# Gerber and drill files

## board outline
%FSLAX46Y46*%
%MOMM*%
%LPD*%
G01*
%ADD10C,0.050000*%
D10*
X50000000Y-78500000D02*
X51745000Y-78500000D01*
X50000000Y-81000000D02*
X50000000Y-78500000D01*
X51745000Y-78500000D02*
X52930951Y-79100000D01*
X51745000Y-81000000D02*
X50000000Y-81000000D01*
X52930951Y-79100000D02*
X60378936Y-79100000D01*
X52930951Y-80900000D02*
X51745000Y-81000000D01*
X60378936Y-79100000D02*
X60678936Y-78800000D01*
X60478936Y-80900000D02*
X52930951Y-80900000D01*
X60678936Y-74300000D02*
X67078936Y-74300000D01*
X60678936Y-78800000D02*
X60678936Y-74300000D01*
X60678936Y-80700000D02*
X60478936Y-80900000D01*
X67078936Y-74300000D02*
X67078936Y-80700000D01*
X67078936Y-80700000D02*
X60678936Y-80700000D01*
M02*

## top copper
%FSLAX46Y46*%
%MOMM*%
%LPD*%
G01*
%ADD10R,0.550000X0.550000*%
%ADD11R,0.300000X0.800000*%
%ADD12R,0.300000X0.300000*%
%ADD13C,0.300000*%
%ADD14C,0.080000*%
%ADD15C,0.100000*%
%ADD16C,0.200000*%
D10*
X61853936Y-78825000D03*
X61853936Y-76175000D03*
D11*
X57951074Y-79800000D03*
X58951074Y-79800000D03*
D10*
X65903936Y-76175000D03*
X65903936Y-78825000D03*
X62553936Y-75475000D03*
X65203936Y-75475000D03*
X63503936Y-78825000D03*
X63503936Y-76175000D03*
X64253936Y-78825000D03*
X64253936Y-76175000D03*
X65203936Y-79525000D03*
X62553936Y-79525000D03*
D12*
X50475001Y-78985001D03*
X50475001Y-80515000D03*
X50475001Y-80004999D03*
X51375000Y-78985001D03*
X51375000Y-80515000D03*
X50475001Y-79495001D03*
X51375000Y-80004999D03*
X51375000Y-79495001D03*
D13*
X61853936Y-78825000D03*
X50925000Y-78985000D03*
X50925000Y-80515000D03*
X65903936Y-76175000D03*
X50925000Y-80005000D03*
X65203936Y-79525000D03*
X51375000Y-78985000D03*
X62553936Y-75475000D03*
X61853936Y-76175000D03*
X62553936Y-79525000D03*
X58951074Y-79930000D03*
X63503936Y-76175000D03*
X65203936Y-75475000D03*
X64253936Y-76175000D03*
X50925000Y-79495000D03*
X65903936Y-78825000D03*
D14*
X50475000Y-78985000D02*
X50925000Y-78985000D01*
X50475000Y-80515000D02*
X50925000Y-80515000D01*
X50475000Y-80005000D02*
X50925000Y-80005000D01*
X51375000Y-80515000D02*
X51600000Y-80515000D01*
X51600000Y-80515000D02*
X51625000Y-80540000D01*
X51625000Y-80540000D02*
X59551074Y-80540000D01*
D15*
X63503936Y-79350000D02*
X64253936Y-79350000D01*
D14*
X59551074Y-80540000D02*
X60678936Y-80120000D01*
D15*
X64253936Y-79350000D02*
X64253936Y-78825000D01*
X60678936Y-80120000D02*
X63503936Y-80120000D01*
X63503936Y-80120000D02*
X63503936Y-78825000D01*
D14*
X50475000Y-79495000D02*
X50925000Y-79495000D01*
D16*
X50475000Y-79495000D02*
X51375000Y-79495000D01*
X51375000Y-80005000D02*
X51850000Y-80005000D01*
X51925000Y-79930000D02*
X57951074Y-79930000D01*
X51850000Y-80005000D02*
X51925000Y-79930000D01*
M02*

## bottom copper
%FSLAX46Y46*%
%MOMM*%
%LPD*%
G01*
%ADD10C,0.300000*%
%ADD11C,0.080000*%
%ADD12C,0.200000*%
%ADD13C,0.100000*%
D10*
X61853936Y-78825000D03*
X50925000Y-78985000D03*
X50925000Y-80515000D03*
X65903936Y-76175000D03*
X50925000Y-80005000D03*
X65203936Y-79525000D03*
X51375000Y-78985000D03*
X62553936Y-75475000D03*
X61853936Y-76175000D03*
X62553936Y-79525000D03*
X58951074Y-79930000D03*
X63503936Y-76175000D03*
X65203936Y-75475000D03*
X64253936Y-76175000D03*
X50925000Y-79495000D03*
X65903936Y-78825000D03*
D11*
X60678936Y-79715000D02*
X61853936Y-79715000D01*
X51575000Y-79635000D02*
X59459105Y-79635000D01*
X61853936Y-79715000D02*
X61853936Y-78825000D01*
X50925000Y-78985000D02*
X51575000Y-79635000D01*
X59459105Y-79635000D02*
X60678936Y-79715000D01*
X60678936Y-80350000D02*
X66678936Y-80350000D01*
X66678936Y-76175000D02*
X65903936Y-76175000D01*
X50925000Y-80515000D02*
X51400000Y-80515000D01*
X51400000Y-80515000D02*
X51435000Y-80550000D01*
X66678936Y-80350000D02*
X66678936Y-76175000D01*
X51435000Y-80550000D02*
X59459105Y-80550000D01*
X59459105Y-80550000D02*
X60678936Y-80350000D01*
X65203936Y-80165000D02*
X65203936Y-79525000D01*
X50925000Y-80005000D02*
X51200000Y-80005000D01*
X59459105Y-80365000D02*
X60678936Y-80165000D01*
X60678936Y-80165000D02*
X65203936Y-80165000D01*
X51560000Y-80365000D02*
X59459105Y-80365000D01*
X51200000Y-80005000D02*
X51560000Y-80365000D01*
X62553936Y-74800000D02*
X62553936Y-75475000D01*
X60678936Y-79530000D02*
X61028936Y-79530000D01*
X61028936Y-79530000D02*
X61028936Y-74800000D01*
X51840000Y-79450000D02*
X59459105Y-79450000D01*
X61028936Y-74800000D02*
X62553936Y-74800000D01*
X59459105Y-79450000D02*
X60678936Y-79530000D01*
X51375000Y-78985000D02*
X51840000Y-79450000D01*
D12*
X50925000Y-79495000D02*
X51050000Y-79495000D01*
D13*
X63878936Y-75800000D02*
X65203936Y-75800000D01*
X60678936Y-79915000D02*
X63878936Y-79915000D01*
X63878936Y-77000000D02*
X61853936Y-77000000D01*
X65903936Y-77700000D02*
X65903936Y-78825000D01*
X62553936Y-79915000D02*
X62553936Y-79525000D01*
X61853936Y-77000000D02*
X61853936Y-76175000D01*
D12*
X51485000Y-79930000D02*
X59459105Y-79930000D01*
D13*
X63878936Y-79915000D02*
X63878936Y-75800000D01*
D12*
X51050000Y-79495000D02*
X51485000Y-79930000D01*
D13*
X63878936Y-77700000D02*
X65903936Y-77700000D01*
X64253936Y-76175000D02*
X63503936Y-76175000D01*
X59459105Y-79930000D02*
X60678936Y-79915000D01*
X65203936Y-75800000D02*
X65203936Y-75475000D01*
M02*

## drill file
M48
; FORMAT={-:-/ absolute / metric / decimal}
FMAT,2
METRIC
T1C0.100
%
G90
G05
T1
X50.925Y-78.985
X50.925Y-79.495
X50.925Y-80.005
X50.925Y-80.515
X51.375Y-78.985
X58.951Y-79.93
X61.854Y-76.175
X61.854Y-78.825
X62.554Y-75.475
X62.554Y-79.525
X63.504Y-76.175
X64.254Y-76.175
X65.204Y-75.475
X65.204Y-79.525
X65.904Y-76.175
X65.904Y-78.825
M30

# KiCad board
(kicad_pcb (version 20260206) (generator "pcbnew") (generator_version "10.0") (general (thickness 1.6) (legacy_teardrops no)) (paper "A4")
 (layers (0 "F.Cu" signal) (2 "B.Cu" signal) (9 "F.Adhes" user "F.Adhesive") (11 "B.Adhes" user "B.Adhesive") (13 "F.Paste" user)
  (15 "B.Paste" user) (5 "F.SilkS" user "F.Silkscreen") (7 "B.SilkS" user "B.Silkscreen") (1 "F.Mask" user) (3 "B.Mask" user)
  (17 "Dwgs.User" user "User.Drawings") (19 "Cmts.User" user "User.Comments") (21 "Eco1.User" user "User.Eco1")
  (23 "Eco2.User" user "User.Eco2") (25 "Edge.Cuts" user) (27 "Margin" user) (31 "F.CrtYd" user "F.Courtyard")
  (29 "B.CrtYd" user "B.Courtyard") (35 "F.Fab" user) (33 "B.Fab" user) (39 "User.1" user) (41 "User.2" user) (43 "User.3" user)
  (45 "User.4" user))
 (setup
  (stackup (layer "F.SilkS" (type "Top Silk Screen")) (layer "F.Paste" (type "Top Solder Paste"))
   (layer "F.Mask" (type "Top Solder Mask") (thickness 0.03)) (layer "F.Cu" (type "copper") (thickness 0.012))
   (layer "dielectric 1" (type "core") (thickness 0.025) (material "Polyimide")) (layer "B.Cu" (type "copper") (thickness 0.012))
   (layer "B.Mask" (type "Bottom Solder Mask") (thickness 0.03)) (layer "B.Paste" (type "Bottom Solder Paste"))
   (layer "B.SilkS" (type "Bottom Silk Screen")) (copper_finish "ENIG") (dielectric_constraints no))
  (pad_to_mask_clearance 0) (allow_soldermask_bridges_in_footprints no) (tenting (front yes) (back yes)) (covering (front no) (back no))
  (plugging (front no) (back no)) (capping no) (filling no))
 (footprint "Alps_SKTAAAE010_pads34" (layer "F.Cu") (at 61.478936 77.5 90)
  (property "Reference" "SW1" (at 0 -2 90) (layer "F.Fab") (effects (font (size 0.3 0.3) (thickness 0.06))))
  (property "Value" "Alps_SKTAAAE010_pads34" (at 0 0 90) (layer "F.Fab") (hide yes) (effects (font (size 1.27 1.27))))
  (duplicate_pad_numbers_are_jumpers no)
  (pad "3" smd rect (at -1.325 0.375 90) (size 0.55 0.55) (layers "F.Cu" "F.Mask") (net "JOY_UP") (solder_mask_margin 0.05)
   (thermal_bridge_angle 45))
  (pad "4" smd rect (at 1.325 0.375 90) (size 0.55 0.55) (layers "F.Cu" "F.Mask") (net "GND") (solder_mask_margin 0.05)
   (thermal_bridge_angle 45)))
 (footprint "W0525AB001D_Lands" (layer "F.Cu") (at 58.451074 79.93)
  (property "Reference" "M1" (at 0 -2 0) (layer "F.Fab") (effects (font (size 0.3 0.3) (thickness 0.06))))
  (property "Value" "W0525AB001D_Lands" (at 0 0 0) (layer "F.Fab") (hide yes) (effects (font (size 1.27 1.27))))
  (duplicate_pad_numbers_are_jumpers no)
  (pad "1" smd rect (at -0.5 -0.13) (size 0.3 0.8) (layers "F.Cu" "F.Mask") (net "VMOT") (solder_mask_margin 0.05) (thermal_bridge_angle 45))
  (pad "2" smd rect (at 0.5 -0.13) (size 0.3 0.8) (layers "F.Cu" "F.Mask") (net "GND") (solder_mask_margin 0.05) (thermal_bridge_angle 45)))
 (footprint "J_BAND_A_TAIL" (layer "F.Cu") (at 50.9 79.75)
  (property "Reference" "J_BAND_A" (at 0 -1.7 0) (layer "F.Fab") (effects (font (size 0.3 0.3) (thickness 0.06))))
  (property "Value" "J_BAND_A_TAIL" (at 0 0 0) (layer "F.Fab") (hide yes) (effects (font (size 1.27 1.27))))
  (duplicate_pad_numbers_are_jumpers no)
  (pad "1" smd rect (at -0.424999 -0.764999) (size 0.3 0.3) (layers "F.Cu" "F.Mask") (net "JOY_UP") (solder_mask_margin 0.05)
   (thermal_bridge_angle 45))
  (pad "2" smd rect (at -0.424999 0.765) (size 0.3 0.3) (layers "F.Cu" "F.Mask") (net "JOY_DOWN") (solder_mask_margin 0.05)
   (thermal_bridge_angle 45))
  (pad "3" smd rect (at -0.424999 0.254999) (size 0.3 0.3) (layers "F.Cu" "F.Mask") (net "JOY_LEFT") (solder_mask_margin 0.05)
   (thermal_bridge_angle 45))
  (pad "4" smd rect (at 0.475 -0.764999) (size 0.3 0.3) (layers "F.Cu" "F.Mask") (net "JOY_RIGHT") (solder_mask_margin 0.05)
   (thermal_bridge_angle 45))
  (pad "5" smd rect (at 0.475 0.765) (size 0.3 0.3) (layers "F.Cu" "F.Mask") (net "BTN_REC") (solder_mask_margin 0.05)
   (thermal_bridge_angle 45))
  (pad "6" smd rect (at -0.424999 -0.254999) (size 0.3 0.3) (layers "F.Cu" "F.Mask") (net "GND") (solder_mask_margin 0.05)
   (thermal_bridge_angle 45))
  (pad "7" smd rect (at 0.475 0.254999) (size 0.3 0.3) (layers "F.Cu" "F.Mask") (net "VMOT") (solder_mask_margin 0.05)
   (thermal_bridge_angle 45))
  (pad "8" smd rect (at 0.475 -0.254999) (size 0.3 0.3) (layers "F.Cu" "F.Mask") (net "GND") (solder_mask_margin 0.05)
   (thermal_bridge_angle 45)))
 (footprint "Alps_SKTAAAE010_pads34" (layer "F.Cu") (at 66.278936 77.5 -90)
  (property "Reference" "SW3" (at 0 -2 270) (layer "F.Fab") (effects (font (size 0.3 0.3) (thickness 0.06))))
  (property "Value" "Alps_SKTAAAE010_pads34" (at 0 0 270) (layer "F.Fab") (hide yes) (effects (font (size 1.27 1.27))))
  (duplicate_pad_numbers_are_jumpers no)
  (pad "3" smd rect (at -1.325 0.375 270) (size 0.55 0.55) (layers "F.Cu" "F.Mask") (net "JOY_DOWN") (solder_mask_margin 0.05)
   (thermal_bridge_angle 45))
  (pad "4" smd rect (at 1.325 0.375 270) (size 0.55 0.55) (layers "F.Cu" "F.Mask") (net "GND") (solder_mask_margin 0.05)
   (thermal_bridge_angle 45)))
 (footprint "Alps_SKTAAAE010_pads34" (layer "F.Cu") (at 63.878936 75.1)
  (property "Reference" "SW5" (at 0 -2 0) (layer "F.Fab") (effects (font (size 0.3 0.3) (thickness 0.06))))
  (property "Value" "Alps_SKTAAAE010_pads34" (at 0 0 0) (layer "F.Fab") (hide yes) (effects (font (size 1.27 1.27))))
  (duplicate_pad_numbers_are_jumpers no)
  (pad "3" smd rect (at -1.325 0.375) (size 0.55 0.55) (layers "F.Cu" "F.Mask") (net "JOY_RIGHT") (solder_mask_margin 0.05)
   (thermal_bridge_angle 45))
  (pad "4" smd rect (at 1.325 0.375) (size 0.55 0.55) (layers "F.Cu" "F.Mask") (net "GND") (solder_mask_margin 0.05)
   (thermal_bridge_angle 45)))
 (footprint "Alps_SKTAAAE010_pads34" (layer "F.Cu") (at 63.878936 79.9 180)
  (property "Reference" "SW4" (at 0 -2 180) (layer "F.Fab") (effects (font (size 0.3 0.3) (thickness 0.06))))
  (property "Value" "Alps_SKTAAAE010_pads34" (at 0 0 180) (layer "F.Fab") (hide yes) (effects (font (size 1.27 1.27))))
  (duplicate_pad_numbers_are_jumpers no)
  (pad "3" smd rect (at -1.325 0.375 180) (size 0.55 0.55) (layers "F.Cu" "F.Mask") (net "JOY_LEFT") (solder_mask_margin 0.05)
   (thermal_bridge_angle 45))
  (pad "4" smd rect (at 1.325 0.375 180) (size 0.55 0.55) (layers "F.Cu" "F.Mask") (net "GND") (solder_mask_margin 0.05)
   (thermal_bridge_angle 45)))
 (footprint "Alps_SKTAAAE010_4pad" (layer "F.Cu") (at 63.878936 77.5 90)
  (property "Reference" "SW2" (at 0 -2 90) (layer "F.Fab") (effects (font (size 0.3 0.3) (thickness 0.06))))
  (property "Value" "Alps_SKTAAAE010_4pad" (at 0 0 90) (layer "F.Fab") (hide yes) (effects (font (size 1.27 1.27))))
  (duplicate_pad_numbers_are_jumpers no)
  (pad "1" smd rect (at -1.325 -0.375 90) (size 0.55 0.55) (layers "F.Cu" "F.Mask") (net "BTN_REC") (solder_mask_margin 0.05)
   (thermal_bridge_angle 45))
  (pad "2" smd rect (at 1.325 -0.375 90) (size 0.55 0.55) (layers "F.Cu" "F.Mask") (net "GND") (solder_mask_margin 0.05)
   (thermal_bridge_angle 45))
  (pad "3" smd rect (at -1.325 0.375 90) (size 0.55 0.55) (layers "F.Cu" "F.Mask") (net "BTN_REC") (solder_mask_margin 0.05)
   (thermal_bridge_angle 45))
  (pad "4" smd rect (at 1.325 0.375 90) (size 0.55 0.55) (layers "F.Cu" "F.Mask") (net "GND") (solder_mask_margin 0.05)
   (thermal_bridge_angle 45)))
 (gr_line (start 50 78.5) (end 51.745 78.5) (stroke (width 0.05) (type default)) (layer "Edge.Cuts"))
 (gr_line (start 50 81) (end 50 78.5) (stroke (width 0.05) (type default)) (layer "Edge.Cuts"))
 (gr_line (start 51.745 78.5) (end 52.930951 79.1) (stroke (width 0.05) (type default)) (layer "Edge.Cuts"))
 (gr_line (start 51.745 81) (end 50 81) (stroke (width 0.05) (type default)) (layer "Edge.Cuts"))
 (gr_line (start 52.930951 79.1) (end 60.378936 79.1) (stroke (width 0.05) (type default)) (layer "Edge.Cuts"))
 (gr_line (start 52.930951 80.9) (end 51.745 81) (stroke (width 0.05) (type default)) (layer "Edge.Cuts"))
 (gr_line (start 60.378936 79.1) (end 60.678936 78.8) (stroke (width 0.05) (type default)) (layer "Edge.Cuts"))
 (gr_line (start 60.478936 80.9) (end 52.930951 80.9) (stroke (width 0.05) (type default)) (layer "Edge.Cuts"))
 (gr_line (start 60.678936 74.3) (end 67.078936 74.3) (stroke (width 0.05) (type default)) (layer "Edge.Cuts"))
 (gr_line (start 60.678936 78.8) (end 60.678936 74.3) (stroke (width 0.05) (type default)) (layer "Edge.Cuts"))
 (gr_line (start 60.678936 80.7) (end 60.478936 80.9) (stroke (width 0.05) (type default)) (layer "Edge.Cuts"))
 (gr_line (start 67.078936 74.3) (end 67.078936 80.7) (stroke (width 0.05) (type default)) (layer "Edge.Cuts"))
 (gr_line (start 67.078936 80.7) (end 60.678936 80.7) (stroke (width 0.05) (type default)) (layer "Edge.Cuts"))
 (segment (start 50.475 78.985) (end 50.925 78.985) (width 0.08) (layer "F.Cu") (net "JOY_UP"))
 (via (at 61.853936 78.825) (size 0.3) (drill 0.1) (layers "F.Cu" "B.Cu") (tenting (front yes) (back yes)) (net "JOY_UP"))
 (via (at 50.925 78.985) (size 0.3) (drill 0.1) (layers "F.Cu" "B.Cu") (tenting (front yes) (back yes)) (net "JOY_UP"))
 (segment (start 51.575 79.635) (end 59.459105 79.635) (width 0.08) (layer "B.Cu") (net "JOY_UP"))
 (segment (start 61.853936 79.715) (end 61.853936 78.825) (width 0.08) (layer "B.Cu") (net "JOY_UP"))
 (segment (start 50.925 78.985) (end 51.575 79.635) (width 0.08) (layer "B.Cu") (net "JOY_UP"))
 (segment (start 60.678936 79.715) (end 61.853936 79.715) (width 0.08) (layer "B.Cu") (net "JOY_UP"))
 (segment (start 59.459105 79.635) (end 60.678936 79.715) (width 0.08) (layer "B.Cu") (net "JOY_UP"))
 (segment (start 50.475 80.515) (end 50.925 80.515) (width 0.08) (layer "F.Cu") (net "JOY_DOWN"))
 (via (at 65.903936 76.175) (size 0.3) (drill 0.1) (layers "F.Cu" "B.Cu") (tenting (front yes) (back yes)) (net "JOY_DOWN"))
 (via (at 50.925 80.515) (size 0.3) (drill 0.1) (layers "F.Cu" "B.Cu") (tenting (front yes) (back yes)) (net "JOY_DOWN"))
 (segment (start 66.678936 80.35) (end 66.678936 76.175) (width 0.08) (layer "B.Cu") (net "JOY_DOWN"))
 (segment (start 60.678936 80.35) (end 66.678936 80.35) (width 0.08) (layer "B.Cu") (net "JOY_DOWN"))
 (segment (start 66.678936 76.175) (end 65.903936 76.175) (width 0.08) (layer "B.Cu") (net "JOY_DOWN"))
 (segment (start 50.925 80.515) (end 51.4 80.515) (width 0.08) (layer "B.Cu") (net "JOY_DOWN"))
 (segment (start 51.435 80.55) (end 59.459105 80.55) (width 0.08) (layer "B.Cu") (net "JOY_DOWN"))
 (segment (start 59.459105 80.55) (end 60.678936 80.35) (width 0.08) (layer "B.Cu") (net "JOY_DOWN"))
 (segment (start 51.4 80.515) (end 51.435 80.55) (width 0.08) (layer "B.Cu") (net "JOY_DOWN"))
 (segment (start 50.475 80.005) (end 50.925 80.005) (width 0.08) (layer "F.Cu") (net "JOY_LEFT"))
 (via (at 50.925 80.005) (size 0.3) (drill 0.1) (layers "F.Cu" "B.Cu") (tenting (front yes) (back yes)) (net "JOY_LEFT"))
 (via (at 65.203936 79.525) (size 0.3) (drill 0.1) (layers "F.Cu" "B.Cu") (tenting (front yes) (back yes)) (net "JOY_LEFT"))
 (segment (start 51.56 80.365) (end 59.459105 80.365) (width 0.08) (layer "B.Cu") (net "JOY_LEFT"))
 (segment (start 51.2 80.005) (end 51.56 80.365) (width 0.08) (layer "B.Cu") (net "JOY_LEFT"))
 (segment (start 60.678936 80.165) (end 65.203936 80.165) (width 0.08) (layer "B.Cu") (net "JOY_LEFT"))
 (segment (start 50.925 80.005) (end 51.2 80.005) (width 0.08) (layer "B.Cu") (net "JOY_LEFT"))
 (segment (start 59.459105 80.365) (end 60.678936 80.165) (width 0.08) (layer "B.Cu") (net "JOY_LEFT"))
 (segment (start 65.203936 80.165) (end 65.203936 79.525) (width 0.08) (layer "B.Cu") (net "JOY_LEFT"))
 (via (at 62.553936 75.475) (size 0.3) (drill 0.1) (layers "F.Cu" "B.Cu") (tenting (front yes) (back yes)) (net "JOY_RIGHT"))
 (via (at 51.375 78.985) (size 0.3) (drill 0.1) (layers "F.Cu" "B.Cu") (tenting (front yes) (back yes)) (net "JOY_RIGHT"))
 (segment (start 62.553936 74.8) (end 62.553936 75.475) (width 0.08) (layer "B.Cu") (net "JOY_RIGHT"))
 (segment (start 59.459105 79.45) (end 60.678936 79.53) (width 0.08) (layer "B.Cu") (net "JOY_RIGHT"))
 (segment (start 61.028936 74.8) (end 62.553936 74.8) (width 0.08) (layer "B.Cu") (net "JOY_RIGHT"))
 (segment (start 51.375 78.985) (end 51.84 79.45) (width 0.08) (layer "B.Cu") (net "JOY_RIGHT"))
 (segment (start 60.678936 79.53) (end 61.028936 79.53) (width 0.08) (layer "B.Cu") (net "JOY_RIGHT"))
 (segment (start 51.84 79.45) (end 59.459105 79.45) (width 0.08) (layer "B.Cu") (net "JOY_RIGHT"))
 (segment (start 61.028936 79.53) (end 61.028936 74.8) (width 0.08) (layer "B.Cu") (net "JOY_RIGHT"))
 (segment (start 51.6 80.515) (end 51.625 80.54) (width 0.08) (layer "F.Cu") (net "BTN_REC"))
 (segment (start 64.253936 79.35) (end 64.253936 78.825) (width 0.1) (layer "F.Cu") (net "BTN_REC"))
 (segment (start 63.503936 79.35) (end 64.253936 79.35) (width 0.1) (layer "F.Cu") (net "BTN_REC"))
 (segment (start 63.503936 80.12) (end 63.503936 78.825) (width 0.1) (layer "F.Cu") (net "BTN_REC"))
 (segment (start 51.375 80.515) (end 51.6 80.515) (width 0.08) (layer "F.Cu") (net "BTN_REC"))
 (segment (start 59.551074 80.54) (end 60.678936 80.12) (width 0.08) (layer "F.Cu") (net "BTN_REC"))
 (segment (start 60.678936 80.12) (end 63.503936 80.12) (width 0.1) (layer "F.Cu") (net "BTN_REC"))
 (segment (start 51.625 80.54) (end 59.551074 80.54) (width 0.08) (layer "F.Cu") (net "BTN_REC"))
 (segment (start 50.475 79.495) (end 51.375 79.495) (width 0.2) (layer "F.Cu") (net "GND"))
 (segment (start 50.475 79.495) (end 50.925 79.495) (width 0.08) (layer "F.Cu") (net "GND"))
 (via (at 64.253936 76.175) (size 0.3) (drill 0.1) (layers "F.Cu" "B.Cu") (tenting (front yes) (back yes)) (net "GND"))
 (via (at 63.503936 76.175) (size 0.3) (drill 0.1) (layers "F.Cu" "B.Cu") (tenting (front yes) (back yes)) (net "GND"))
 (via (at 65.203936 75.475) (size 0.3) (drill 0.1) (layers "F.Cu" "B.Cu") (tenting (front yes) (back yes)) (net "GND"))
 (via (at 50.925 79.495) (size 0.3) (drill 0.1) (layers "F.Cu" "B.Cu") (tenting (front yes) (back yes)) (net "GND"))
 (via (at 61.853936 76.175) (size 0.3) (drill 0.1) (layers "F.Cu" "B.Cu") (tenting (front yes) (back yes)) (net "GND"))
 (via (at 58.951074 79.93) (size 0.3) (drill 0.1) (layers "F.Cu" "B.Cu") (tenting (front yes) (back yes)) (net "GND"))
 (via (at 62.553936 79.525) (size 0.3) (drill 0.1) (layers "F.Cu" "B.Cu") (tenting (front yes) (back yes)) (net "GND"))
 (via (at 65.903936 78.825) (size 0.3) (drill 0.1) (layers "F.Cu" "B.Cu") (tenting (front yes) (back yes)) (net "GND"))
 (segment (start 59.459105 79.93) (end 60.678936 79.915) (width 0.1) (layer "B.Cu") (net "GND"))
 (segment (start 65.203936 75.8) (end 65.203936 75.475) (width 0.1) (layer "B.Cu") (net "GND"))
 (segment (start 51.485 79.93) (end 59.459105 79.93) (width 0.2) (layer "B.Cu") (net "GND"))
 (segment (start 62.553936 79.915) (end 62.553936 79.525) (width 0.1) (layer "B.Cu") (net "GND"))
 (segment (start 63.878936 75.8) (end 65.203936 75.8) (width 0.1) (layer "B.Cu") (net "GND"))
 (segment (start 61.853936 77) (end 61.853936 76.175) (width 0.1) (layer "B.Cu") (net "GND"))
 (segment (start 60.678936 79.915) (end 63.878936 79.915) (width 0.1) (layer "B.Cu") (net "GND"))
 (segment (start 63.878936 77.7) (end 65.903936 77.7) (width 0.1) (layer "B.Cu") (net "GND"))
 (segment (start 63.878936 77) (end 61.853936 77) (width 0.1) (layer "B.Cu") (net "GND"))
 (segment (start 63.878936 79.915) (end 63.878936 75.8) (width 0.1) (layer "B.Cu") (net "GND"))
 (segment (start 51.05 79.495) (end 51.485 79.93) (width 0.2) (layer "B.Cu") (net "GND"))
 (segment (start 50.925 79.495) (end 51.05 79.495) (width 0.2) (layer "B.Cu") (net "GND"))
 (segment (start 65.903936 77.7) (end 65.903936 78.825) (width 0.1) (layer "B.Cu") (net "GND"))
 (segment (start 64.253936 76.175) (end 63.503936 76.175) (width 0.1) (layer "B.Cu") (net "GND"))
 (segment (start 51.375 80.005) (end 51.85 80.005) (width 0.2) (layer "F.Cu") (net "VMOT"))
 (segment (start 51.925 79.93) (end 57.951074 79.93) (width 0.2) (layer "F.Cu") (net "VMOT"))
 (segment (start 51.85 80.005) (end 51.925 79.93) (width 0.2) (layer "F.Cu") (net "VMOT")))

